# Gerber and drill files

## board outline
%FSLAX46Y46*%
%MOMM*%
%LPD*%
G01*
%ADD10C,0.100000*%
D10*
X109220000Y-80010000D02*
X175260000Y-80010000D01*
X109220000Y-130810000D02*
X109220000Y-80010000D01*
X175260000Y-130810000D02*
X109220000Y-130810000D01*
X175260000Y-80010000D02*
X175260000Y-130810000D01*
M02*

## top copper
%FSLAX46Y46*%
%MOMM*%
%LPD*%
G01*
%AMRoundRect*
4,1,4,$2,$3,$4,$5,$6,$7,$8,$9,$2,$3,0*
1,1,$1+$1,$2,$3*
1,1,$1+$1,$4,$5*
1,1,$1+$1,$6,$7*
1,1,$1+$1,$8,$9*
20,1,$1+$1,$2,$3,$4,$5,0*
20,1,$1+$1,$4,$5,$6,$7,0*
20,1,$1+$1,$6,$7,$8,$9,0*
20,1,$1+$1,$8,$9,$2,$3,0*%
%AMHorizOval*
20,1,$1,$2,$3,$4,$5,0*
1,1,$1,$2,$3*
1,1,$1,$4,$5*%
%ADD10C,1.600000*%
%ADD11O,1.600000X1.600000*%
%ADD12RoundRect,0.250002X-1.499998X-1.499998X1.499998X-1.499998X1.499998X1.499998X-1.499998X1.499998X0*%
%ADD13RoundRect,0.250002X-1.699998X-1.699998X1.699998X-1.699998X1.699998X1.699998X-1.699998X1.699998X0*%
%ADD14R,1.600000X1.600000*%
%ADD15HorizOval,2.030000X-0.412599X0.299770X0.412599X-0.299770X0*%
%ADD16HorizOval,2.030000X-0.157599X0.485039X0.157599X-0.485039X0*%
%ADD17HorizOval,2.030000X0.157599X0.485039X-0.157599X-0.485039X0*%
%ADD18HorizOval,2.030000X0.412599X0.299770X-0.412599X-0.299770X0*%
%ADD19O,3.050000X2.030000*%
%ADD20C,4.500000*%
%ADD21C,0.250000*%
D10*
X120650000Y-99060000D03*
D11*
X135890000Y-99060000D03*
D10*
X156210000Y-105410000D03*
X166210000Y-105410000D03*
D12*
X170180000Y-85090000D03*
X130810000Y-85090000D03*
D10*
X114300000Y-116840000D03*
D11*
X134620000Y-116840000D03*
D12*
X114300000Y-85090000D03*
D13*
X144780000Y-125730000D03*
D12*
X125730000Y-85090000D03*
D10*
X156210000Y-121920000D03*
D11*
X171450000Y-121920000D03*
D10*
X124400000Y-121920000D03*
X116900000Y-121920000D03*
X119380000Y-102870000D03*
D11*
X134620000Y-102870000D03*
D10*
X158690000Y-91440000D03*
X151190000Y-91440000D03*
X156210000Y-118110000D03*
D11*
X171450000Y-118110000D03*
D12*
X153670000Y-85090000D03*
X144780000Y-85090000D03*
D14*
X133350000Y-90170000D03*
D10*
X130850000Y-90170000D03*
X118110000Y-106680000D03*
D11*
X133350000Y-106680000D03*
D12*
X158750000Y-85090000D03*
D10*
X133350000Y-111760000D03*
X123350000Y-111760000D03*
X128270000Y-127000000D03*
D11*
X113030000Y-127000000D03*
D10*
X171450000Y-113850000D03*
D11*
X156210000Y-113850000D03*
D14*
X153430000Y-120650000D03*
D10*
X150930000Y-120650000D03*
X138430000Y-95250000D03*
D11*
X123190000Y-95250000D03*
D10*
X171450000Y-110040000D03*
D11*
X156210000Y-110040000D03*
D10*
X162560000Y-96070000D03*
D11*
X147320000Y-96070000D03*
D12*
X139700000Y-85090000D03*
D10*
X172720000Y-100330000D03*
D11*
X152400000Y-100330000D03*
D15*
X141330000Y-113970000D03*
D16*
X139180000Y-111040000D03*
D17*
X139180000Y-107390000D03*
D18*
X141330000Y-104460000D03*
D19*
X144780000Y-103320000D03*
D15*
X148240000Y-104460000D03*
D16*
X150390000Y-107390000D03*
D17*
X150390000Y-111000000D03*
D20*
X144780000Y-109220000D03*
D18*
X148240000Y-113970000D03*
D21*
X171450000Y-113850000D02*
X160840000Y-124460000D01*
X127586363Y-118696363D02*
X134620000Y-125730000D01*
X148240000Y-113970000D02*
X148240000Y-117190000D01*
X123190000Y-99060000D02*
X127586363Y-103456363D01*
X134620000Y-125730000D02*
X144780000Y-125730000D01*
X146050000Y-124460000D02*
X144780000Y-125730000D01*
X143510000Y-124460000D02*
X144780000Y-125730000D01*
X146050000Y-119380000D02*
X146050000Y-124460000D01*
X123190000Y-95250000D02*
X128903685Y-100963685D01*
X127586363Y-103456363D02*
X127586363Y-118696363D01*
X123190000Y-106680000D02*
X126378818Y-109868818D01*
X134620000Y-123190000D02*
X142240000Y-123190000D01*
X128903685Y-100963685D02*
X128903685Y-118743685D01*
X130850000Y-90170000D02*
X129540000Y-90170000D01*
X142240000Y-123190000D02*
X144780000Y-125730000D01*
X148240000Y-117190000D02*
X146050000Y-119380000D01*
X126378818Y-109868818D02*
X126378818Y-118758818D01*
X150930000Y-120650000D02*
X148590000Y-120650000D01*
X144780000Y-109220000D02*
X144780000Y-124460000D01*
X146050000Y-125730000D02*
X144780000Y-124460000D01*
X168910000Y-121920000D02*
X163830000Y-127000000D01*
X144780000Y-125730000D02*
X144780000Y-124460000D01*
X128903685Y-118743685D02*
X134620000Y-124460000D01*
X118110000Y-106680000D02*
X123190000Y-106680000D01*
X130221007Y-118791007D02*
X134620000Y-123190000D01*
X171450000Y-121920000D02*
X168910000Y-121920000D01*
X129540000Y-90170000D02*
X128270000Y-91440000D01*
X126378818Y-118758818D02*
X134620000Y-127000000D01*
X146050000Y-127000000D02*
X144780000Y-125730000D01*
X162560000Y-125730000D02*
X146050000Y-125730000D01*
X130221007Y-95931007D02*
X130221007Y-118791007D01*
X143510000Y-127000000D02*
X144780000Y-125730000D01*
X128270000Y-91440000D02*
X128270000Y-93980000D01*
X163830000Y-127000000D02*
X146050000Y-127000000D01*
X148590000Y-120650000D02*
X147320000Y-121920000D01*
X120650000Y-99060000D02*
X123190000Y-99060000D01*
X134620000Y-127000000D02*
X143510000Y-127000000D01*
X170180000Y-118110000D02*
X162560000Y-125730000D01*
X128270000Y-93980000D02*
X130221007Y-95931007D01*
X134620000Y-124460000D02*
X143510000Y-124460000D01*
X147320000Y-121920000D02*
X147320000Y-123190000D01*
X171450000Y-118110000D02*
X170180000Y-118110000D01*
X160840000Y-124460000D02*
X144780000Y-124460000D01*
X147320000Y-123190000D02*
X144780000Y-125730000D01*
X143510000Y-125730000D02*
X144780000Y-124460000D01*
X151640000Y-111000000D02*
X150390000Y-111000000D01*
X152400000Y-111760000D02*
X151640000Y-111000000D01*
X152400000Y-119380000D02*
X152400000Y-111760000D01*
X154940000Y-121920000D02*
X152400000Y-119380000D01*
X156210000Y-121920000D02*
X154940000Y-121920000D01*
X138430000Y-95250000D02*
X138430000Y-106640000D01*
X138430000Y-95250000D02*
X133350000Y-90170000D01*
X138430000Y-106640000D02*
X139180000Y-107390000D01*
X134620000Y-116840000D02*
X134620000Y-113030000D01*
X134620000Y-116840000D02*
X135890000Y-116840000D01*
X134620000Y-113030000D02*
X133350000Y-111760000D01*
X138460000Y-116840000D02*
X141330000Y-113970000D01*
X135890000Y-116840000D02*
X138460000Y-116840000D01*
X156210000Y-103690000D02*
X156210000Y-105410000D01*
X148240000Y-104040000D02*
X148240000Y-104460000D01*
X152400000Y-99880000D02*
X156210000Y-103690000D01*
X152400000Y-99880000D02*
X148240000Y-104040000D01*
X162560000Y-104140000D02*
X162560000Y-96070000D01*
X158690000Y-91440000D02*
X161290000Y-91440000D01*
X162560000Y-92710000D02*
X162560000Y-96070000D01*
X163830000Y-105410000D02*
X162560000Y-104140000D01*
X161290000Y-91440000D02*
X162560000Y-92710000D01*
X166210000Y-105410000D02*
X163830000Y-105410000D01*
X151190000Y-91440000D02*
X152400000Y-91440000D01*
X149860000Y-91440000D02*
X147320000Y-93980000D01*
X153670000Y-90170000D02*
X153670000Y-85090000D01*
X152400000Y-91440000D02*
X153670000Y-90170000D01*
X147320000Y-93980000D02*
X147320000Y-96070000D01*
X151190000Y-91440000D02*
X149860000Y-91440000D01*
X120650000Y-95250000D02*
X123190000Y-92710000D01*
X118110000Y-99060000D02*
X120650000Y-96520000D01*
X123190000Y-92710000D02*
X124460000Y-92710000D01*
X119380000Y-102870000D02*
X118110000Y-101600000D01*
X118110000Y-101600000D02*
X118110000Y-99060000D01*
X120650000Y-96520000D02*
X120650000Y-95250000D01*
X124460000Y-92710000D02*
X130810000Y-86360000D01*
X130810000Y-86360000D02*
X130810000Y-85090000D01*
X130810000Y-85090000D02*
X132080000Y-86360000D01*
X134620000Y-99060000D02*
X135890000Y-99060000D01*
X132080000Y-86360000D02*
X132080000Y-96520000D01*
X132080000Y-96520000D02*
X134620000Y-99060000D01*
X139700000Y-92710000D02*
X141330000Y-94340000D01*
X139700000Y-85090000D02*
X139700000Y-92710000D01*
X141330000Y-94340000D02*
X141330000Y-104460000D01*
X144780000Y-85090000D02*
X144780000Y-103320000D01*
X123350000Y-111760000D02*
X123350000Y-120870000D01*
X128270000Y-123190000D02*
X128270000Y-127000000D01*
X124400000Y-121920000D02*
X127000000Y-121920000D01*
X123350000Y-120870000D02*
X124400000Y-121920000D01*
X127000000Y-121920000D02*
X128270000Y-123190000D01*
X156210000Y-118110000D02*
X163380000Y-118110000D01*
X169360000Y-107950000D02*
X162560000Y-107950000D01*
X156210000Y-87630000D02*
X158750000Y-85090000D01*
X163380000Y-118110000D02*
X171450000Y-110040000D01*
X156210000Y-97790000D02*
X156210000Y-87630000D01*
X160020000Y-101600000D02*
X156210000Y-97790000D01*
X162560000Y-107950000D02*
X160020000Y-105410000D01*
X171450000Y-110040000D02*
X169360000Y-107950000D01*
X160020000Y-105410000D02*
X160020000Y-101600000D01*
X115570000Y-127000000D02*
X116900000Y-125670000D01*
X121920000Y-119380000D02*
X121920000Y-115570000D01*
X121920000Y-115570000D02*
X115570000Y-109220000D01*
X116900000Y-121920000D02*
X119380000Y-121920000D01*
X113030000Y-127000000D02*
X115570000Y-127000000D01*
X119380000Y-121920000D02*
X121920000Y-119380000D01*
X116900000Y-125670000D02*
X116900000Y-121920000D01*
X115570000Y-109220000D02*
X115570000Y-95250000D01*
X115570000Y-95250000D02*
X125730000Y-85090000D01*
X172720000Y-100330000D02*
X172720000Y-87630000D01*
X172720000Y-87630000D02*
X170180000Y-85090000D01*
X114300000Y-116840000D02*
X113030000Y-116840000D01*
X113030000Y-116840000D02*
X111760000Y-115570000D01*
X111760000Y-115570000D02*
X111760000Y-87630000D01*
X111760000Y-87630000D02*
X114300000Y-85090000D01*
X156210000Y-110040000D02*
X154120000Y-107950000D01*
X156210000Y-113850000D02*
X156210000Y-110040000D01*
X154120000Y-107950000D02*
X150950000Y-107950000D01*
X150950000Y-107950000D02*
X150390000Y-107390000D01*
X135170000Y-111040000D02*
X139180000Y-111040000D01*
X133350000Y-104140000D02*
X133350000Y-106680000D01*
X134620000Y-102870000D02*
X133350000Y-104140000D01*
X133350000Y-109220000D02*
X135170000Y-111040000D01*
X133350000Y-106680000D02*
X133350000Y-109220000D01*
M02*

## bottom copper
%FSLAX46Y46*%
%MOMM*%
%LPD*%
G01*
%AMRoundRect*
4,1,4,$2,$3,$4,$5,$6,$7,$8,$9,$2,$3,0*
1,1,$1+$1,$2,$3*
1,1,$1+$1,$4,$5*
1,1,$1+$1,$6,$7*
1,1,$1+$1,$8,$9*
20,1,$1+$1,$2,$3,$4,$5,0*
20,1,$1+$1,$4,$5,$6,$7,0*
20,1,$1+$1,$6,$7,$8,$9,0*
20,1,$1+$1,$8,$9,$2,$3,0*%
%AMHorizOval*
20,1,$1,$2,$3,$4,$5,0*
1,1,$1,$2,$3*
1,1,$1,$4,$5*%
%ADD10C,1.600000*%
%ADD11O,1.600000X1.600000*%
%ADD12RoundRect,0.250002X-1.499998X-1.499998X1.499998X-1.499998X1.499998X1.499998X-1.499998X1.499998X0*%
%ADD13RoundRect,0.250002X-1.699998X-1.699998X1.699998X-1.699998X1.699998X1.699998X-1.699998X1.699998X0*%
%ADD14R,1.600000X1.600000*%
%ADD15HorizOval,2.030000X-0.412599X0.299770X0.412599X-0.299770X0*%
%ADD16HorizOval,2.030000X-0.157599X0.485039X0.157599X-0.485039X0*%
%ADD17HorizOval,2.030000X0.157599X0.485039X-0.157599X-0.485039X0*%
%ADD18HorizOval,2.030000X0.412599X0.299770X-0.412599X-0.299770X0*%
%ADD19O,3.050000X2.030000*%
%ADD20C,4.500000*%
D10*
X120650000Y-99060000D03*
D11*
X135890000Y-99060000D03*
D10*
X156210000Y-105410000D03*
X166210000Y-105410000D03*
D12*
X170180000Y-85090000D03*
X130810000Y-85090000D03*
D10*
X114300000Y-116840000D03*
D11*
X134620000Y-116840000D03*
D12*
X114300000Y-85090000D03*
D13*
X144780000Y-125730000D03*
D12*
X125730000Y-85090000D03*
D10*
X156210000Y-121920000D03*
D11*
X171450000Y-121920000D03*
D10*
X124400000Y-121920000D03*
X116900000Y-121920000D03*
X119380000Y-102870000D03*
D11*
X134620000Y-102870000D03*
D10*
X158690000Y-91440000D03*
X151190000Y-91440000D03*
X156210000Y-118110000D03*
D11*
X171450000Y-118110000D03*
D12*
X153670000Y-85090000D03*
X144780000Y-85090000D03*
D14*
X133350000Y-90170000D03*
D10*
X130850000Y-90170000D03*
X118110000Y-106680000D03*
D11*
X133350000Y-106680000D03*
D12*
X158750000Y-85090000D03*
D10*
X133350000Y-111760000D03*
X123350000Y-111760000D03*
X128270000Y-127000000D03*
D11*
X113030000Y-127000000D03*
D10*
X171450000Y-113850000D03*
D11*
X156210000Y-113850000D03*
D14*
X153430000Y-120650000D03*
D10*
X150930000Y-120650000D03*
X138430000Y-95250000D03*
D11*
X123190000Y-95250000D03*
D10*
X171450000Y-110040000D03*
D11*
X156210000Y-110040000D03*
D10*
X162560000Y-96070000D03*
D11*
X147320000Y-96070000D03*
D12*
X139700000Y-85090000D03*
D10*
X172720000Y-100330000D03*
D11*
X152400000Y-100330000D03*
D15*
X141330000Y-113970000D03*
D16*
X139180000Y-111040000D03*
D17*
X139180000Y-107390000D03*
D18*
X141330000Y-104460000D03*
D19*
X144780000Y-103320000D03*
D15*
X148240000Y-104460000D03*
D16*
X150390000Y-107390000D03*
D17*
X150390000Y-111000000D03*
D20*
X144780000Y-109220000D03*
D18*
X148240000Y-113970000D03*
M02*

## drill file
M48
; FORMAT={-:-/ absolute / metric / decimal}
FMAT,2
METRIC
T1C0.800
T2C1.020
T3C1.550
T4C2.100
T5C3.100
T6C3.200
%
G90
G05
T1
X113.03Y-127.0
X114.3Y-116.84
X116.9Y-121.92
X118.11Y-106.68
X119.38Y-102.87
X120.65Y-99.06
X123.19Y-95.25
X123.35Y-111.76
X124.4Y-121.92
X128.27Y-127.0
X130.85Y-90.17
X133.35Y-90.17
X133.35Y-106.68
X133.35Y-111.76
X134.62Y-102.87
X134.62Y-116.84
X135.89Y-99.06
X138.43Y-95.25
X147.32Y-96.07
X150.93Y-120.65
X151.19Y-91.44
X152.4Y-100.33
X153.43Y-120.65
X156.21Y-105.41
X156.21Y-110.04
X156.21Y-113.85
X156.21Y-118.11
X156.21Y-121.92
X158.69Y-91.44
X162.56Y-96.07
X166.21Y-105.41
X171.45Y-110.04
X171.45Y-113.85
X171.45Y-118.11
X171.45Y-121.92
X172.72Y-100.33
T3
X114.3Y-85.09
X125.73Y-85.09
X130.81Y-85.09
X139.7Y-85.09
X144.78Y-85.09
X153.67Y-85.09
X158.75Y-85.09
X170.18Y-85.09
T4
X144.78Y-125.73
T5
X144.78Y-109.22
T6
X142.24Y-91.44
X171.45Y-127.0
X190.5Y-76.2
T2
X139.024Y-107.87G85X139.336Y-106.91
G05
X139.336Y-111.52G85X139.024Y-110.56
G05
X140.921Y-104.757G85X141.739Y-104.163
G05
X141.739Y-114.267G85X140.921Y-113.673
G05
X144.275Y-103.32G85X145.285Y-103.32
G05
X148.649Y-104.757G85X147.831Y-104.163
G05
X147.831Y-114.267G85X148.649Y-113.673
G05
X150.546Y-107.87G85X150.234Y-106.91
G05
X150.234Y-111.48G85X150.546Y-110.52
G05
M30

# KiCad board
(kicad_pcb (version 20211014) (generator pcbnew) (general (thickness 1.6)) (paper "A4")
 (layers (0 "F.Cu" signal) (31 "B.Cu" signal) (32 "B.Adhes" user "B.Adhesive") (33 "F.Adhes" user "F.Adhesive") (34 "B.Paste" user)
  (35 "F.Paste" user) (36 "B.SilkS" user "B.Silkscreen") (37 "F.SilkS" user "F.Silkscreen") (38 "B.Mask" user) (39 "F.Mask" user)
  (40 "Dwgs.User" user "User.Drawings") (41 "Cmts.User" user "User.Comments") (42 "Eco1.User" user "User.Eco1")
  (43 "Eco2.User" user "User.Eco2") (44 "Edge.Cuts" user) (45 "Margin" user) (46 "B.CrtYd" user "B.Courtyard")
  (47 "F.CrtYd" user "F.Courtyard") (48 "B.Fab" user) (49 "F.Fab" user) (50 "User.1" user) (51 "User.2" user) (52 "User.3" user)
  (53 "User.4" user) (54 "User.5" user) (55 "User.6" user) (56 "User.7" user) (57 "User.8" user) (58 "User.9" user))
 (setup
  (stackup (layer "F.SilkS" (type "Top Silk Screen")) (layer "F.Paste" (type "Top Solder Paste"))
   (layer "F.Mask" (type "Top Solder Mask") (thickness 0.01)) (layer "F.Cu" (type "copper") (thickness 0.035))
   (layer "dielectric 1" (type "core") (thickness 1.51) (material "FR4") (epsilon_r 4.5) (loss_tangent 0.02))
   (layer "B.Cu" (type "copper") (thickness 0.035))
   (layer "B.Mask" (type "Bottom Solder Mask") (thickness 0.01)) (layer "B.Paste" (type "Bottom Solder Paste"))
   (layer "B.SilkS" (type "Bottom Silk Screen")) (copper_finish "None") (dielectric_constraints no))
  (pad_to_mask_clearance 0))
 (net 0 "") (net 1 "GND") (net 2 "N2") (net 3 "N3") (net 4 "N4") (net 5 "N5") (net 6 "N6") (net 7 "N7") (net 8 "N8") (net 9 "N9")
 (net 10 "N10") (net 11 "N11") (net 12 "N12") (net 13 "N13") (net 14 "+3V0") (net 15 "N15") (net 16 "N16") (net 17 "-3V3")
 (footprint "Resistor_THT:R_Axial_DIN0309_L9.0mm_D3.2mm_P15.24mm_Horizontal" (layer "F.Cu") (at 120.65 99.06)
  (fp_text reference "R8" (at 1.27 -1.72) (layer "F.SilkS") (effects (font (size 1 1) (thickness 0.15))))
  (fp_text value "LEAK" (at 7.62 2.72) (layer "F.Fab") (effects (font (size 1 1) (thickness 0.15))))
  (pad "1" thru_hole circle (at 0 0) (size 1.6 1.6) (drill 0.8) (layers *.Cu *.Mask) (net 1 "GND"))
  (pad "2" thru_hole oval (at 15.24 0) (size 1.6 1.6) (drill 0.8) (layers *.Cu *.Mask) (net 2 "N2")))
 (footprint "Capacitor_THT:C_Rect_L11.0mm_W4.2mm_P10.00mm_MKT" (layer "F.Cu") (at 156.21 105.41)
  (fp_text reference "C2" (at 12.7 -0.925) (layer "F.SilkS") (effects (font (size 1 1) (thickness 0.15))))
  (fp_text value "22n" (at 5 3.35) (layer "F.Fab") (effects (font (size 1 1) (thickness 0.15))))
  (pad "1" thru_hole circle (at 0 0) (size 1.6 1.6) (drill 0.8) (layers *.Cu *.Mask) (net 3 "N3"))
  (pad "2" thru_hole circle (at 10 0) (size 1.6 1.6) (drill 0.8) (layers *.Cu *.Mask) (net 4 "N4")))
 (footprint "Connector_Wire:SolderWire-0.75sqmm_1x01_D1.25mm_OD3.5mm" (layer "F.Cu") (at 170.18 85.09)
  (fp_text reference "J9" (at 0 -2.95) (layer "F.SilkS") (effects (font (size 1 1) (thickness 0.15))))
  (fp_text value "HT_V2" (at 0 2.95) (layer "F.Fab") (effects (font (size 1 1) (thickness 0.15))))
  (pad "1" thru_hole roundrect (at 0 0) (size 3.5 3.5) (drill 1.55) (layers *.Cu *.Mask) (roundrect_rratio 0.071429) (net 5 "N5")))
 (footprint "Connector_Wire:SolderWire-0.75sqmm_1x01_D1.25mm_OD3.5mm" (layer "F.Cu") (at 130.81 85.09)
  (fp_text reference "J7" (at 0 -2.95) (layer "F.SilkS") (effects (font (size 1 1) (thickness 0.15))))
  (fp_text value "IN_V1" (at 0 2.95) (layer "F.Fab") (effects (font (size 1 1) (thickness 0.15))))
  (pad "1" thru_hole roundrect (at 0 0) (size 3.5 3.5) (drill 1.55) (layers *.Cu *.Mask) (roundrect_rratio 0.071429) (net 2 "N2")))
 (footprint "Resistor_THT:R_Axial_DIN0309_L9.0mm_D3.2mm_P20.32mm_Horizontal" (layer "F.Cu") (at 114.3 116.84)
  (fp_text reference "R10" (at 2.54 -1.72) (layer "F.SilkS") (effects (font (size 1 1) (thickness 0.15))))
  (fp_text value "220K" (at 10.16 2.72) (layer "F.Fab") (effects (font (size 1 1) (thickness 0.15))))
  (pad "1" thru_hole circle (at 0 0) (size 1.6 1.6) (drill 0.8) (layers *.Cu *.Mask) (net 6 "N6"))
  (pad "2" thru_hole oval (at 20.32 0) (size 1.6 1.6) (drill 0.8) (layers *.Cu *.Mask) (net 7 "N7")))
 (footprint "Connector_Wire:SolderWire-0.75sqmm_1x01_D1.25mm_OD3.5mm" (layer "F.Cu") (at 114.3 85.09)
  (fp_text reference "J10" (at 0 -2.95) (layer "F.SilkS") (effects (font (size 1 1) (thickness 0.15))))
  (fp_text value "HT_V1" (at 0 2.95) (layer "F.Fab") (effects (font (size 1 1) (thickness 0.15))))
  (pad "1" thru_hole roundrect (at 0 0) (size 3.5 3.5) (drill 1.55) (layers *.Cu *.Mask) (roundrect_rratio 0.071429) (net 6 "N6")))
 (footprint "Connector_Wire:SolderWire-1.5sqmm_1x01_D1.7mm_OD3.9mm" (layer "F.Cu") (at 144.78 125.73)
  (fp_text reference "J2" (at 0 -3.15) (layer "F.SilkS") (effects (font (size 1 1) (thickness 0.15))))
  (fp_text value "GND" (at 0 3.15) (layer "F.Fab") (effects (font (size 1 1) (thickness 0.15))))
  (pad "1" thru_hole roundrect (at 0 0) (size 3.9 3.9) (drill 2.1) (layers *.Cu *.Mask) (roundrect_rratio 0.064103) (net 1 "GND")))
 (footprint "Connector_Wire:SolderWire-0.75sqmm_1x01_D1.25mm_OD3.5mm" (layer "F.Cu") (at 125.73 85.09)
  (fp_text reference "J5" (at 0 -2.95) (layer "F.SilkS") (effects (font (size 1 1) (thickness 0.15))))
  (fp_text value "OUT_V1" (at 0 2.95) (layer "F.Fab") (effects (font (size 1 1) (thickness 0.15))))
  (pad "1" thru_hole roundrect (at 0 0) (size 3.5 3.5) (drill 1.55) (layers *.Cu *.Mask) (roundrect_rratio 0.071429) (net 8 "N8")))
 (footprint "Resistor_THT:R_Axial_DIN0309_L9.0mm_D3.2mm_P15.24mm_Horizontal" (layer "F.Cu") (at 156.21 121.92)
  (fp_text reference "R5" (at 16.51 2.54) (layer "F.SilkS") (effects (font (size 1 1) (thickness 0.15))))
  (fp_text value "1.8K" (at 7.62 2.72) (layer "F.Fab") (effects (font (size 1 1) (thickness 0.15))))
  (pad "1" thru_hole circle (at 0 0) (size 1.6 1.6) (drill 0.8) (layers *.Cu *.Mask) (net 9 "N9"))
  (pad "2" thru_hole oval (at 15.24 0) (size 1.6 1.6) (drill 0.8) (layers *.Cu *.Mask) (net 1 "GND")))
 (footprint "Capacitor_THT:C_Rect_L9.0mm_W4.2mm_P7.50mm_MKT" (layer "F.Cu") (at 124.4 121.92 180)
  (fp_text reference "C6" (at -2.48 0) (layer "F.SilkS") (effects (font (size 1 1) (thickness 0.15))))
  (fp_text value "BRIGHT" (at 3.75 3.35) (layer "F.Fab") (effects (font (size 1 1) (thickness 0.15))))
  (pad "1" thru_hole circle (at 0 0 180) (size 1.6 1.6) (drill 0.8) (layers *.Cu *.Mask) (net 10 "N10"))
  (pad "2" thru_hole circle (at 7.5 0 180) (size 1.6 1.6) (drill 0.8) (layers *.Cu *.Mask) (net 8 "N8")))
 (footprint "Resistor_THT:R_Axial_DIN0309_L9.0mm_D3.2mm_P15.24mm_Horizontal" (layer "F.Cu") (at 119.38 102.87)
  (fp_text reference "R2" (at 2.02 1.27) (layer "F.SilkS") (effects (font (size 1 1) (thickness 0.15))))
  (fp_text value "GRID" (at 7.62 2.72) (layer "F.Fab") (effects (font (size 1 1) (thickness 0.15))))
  (pad "1" thru_hole circle (at 0 0) (size 1.6 1.6) (drill 0.8) (layers *.Cu *.Mask) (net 2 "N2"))
  (pad "2" thru_hole oval (at 15.24 0) (size 1.6 1.6) (drill 0.8) (layers *.Cu *.Mask) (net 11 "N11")))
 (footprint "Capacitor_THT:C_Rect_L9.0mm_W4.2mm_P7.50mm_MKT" (layer "F.Cu") (at 158.69 91.44 180)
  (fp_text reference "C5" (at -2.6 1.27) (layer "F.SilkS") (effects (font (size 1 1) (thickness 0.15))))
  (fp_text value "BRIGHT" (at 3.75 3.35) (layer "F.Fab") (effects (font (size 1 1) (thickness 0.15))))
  (pad "1" thru_hole circle (at 0 0 180) (size 1.6 1.6) (drill 0.8) (layers *.Cu *.Mask) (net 4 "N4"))
  (pad "2" thru_hole circle (at 7.5 0 180) (size 1.6 1.6) (drill 0.8) (layers *.Cu *.Mask) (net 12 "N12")))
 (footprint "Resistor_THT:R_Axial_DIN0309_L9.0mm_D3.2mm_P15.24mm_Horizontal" (layer "F.Cu") (at 156.21 118.11)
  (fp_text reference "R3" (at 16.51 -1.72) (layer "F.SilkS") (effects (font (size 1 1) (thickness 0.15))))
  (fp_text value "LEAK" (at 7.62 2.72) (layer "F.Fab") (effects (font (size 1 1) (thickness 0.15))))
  (pad "1" thru_hole circle (at 0 0) (size 1.6 1.6) (drill 0.8) (layers *.Cu *.Mask) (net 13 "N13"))
  (pad "2" thru_hole oval (at 15.24 0) (size 1.6 1.6) (drill 0.8) (layers *.Cu *.Mask) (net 1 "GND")))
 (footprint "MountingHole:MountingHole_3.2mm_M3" (layer "F.Cu") (at 171.45 127)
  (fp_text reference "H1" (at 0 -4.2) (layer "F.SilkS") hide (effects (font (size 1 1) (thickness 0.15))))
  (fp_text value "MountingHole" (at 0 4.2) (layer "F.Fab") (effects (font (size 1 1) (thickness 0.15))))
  (pad "" np_thru_hole circle (at 0 0) (size 3.2 3.2) (drill 3.2) (layers *.Cu *.Mask)))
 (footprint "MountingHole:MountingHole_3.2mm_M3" (layer "F.Cu") (at 190.5 76.2)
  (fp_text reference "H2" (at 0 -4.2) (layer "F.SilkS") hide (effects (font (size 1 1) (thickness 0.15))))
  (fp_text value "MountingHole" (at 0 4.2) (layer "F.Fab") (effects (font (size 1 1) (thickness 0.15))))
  (pad "" np_thru_hole circle (at 0 0) (size 3.2 3.2) (drill 3.2) (layers *.Cu *.Mask)))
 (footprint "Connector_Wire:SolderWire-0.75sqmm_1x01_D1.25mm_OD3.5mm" (layer "F.Cu") (at 153.67 85.09)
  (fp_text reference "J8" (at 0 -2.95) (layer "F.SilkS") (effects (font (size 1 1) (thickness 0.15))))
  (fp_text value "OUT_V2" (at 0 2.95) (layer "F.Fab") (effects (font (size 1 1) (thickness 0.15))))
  (pad "1" thru_hole roundrect (at 0 0) (size 3.5 3.5) (drill 1.55) (layers *.Cu *.Mask) (roundrect_rratio 0.071429) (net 12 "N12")))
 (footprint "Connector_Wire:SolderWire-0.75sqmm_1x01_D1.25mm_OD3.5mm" (layer "F.Cu") (at 144.78 85.09)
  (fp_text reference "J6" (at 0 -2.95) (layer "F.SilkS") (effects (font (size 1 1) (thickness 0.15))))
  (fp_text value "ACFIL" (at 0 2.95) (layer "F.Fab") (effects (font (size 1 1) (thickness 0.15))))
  (pad "1" thru_hole roundrect (at 0 0) (size 3.5 3.5) (drill 1.55) (layers *.Cu *.Mask) (roundrect_rratio 0.071429) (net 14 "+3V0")))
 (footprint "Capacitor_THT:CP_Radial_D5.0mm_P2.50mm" (layer "F.Cu") (at 133.35 90.17 180)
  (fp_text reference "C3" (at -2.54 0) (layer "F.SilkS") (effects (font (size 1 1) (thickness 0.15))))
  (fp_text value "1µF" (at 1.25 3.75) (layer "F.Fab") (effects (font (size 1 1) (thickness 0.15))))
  (pad "1" thru_hole rect (at 0 0 180) (size 1.6 1.6) (drill 0.8) (layers *.Cu *.Mask) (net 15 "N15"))
  (pad "2" thru_hole circle (at 2.5 0 180) (size 1.6 1.6) (drill 0.8) (layers *.Cu *.Mask) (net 1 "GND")))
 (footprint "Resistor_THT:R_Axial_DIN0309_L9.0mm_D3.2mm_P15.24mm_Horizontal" (layer "F.Cu") (at 118.11 106.68)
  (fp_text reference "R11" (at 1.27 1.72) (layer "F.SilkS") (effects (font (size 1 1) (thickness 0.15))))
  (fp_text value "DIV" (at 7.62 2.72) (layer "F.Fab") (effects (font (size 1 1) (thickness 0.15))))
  (pad "1" thru_hole circle (at 0 0) (size 1.6 1.6) (drill 0.8) (layers *.Cu *.Mask) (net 1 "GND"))
  (pad "2" thru_hole oval (at 15.24 0) (size 1.6 1.6) (drill 0.8) (layers *.Cu *.Mask) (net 11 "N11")))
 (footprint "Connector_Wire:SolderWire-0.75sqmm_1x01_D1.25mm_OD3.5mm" (layer "F.Cu") (at 158.75 85.09)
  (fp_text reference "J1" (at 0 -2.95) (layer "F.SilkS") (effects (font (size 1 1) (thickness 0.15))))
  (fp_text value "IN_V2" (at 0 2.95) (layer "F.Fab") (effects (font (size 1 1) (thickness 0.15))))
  (pad "1" thru_hole roundrect (at 0 0) (size 3.5 3.5) (drill 1.55) (layers *.Cu *.Mask) (roundrect_rratio 0.071429) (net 13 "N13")))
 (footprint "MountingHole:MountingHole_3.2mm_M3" (layer "F.Cu") (at 142.24 91.44)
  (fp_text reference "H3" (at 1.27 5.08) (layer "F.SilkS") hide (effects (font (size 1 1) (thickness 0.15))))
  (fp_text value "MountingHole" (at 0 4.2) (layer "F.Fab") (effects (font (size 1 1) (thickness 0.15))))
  (pad "" np_thru_hole circle (at 0 0) (size 3.2 3.2) (drill 3.2) (layers *.Cu *.Mask)))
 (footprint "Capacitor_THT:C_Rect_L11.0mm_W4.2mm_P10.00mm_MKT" (layer "F.Cu") (at 133.35 111.76 180)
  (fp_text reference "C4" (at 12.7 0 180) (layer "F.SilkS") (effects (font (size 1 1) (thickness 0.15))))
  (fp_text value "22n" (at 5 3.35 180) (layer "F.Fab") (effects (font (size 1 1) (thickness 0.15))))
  (pad "1" thru_hole circle (at 0 0 180) (size 1.6 1.6) (drill 0.8) (layers *.Cu *.Mask) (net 7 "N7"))
  (pad "2" thru_hole circle (at 10 0 180) (size 1.6 1.6) (drill 0.8) (layers *.Cu *.Mask) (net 10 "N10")))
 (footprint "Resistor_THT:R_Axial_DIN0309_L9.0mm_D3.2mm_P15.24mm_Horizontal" (layer "F.Cu") (at 128.27 127 180)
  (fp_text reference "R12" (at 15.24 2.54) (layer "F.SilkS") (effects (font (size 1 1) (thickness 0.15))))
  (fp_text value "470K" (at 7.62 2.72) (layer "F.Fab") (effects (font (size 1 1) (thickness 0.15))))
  (pad "1" thru_hole circle (at 0 0 180) (size 1.6 1.6) (drill 0.8) (layers *.Cu *.Mask) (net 10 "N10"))
  (pad "2" thru_hole oval (at 15.24 0 180) (size 1.6 1.6) (drill 0.8) (layers *.Cu *.Mask) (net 8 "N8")))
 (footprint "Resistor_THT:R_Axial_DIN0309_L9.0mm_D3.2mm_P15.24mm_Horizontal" (layer "F.Cu") (at 171.45 113.85 180)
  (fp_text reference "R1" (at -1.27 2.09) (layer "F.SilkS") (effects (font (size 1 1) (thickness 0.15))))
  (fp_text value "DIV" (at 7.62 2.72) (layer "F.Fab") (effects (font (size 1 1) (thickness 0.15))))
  (pad "1" thru_hole circle (at 0 0 180) (size 1.6 1.6) (drill 0.8) (layers *.Cu *.Mask) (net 1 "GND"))
  (pad "2" thru_hole oval (at 15.24 0 180) (size 1.6 1.6) (drill 0.8) (layers *.Cu *.Mask) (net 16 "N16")))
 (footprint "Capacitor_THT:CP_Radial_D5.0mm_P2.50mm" (layer "F.Cu") (at 153.43 120.65 180)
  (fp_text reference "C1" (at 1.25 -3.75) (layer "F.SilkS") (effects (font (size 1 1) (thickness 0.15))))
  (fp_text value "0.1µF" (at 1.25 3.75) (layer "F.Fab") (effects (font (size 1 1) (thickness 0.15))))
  (pad "1" thru_hole rect (at 0 0 180) (size 1.6 1.6) (drill 0.8) (layers *.Cu *.Mask) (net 9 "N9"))
  (pad "2" thru_hole circle (at 2.5 0 180) (size 1.6 1.6) (drill 0.8) (layers *.Cu *.Mask) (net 1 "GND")))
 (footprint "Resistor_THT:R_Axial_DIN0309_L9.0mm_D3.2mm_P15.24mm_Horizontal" (layer "F.Cu") (at 138.43 95.25 180)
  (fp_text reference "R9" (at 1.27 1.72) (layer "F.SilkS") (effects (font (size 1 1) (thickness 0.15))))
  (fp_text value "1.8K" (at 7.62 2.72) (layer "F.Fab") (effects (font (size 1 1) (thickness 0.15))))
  (pad "1" thru_hole circle (at 0 0 180) (size 1.6 1.6) (drill 0.8) (layers *.Cu *.Mask) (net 15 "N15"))
  (pad "2" thru_hole oval (at 15.24 0 180) (size 1.6 1.6) (drill 0.8) (layers *.Cu *.Mask) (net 1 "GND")))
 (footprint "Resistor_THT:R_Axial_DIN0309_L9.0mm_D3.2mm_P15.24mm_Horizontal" (layer "F.Cu") (at 171.45 110.04 180)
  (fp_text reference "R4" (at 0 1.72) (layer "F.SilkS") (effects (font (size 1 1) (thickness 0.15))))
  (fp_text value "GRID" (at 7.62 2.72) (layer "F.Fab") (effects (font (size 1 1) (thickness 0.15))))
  (pad "1" thru_hole circle (at 0 0 180) (size 1.6 1.6) (drill 0.8) (layers *.Cu *.Mask) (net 13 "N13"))
  (pad "2" thru_hole oval (at 15.24 0 180) (size 1.6 1.6) (drill 0.8) (layers *.Cu *.Mask) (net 16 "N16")))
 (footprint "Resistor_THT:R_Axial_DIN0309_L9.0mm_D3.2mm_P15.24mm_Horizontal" (layer "F.Cu") (at 162.56 96.07 180)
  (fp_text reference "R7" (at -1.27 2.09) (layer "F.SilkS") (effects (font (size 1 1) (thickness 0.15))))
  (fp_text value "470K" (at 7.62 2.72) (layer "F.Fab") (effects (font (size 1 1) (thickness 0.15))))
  (pad "1" thru_hole circle (at 0 0 180) (size 1.6 1.6) (drill 0.8) (layers *.Cu *.Mask) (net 4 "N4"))
  (pad "2" thru_hole oval (at 15.24 0 180) (size 1.6 1.6) (drill 0.8) (layers *.Cu *.Mask) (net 12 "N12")))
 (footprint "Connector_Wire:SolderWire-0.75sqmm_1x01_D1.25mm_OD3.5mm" (layer "F.Cu") (at 139.7 85.09)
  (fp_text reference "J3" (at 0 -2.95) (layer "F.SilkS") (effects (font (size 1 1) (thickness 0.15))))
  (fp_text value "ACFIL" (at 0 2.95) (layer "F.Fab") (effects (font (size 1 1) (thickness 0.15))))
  (pad "1" thru_hole roundrect (at 0 0) (size 3.5 3.5) (drill 1.55) (layers *.Cu *.Mask) (roundrect_rratio 0.071429) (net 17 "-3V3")))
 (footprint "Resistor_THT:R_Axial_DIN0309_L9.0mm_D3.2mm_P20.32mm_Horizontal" (layer "F.Cu") (at 172.72 100.33 180)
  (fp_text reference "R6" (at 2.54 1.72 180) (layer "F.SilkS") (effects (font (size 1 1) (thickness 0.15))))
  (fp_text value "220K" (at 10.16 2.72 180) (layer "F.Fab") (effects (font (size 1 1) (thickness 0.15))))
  (pad "1" thru_hole circle (at 0 0 180) (size 1.6 1.6) (drill 0.8) (layers *.Cu *.Mask) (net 5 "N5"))
  (pad "2" thru_hole oval (at 20.32 0 180) (size 1.6 1.6) (drill 0.8) (layers *.Cu *.Mask) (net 3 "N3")))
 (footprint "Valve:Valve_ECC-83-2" (layer "B.Cu") (at 141.33 113.97 180)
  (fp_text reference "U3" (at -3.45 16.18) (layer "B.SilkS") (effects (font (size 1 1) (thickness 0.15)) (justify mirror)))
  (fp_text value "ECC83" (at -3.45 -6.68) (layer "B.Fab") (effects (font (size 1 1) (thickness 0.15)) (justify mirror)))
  (pad "1" thru_hole oval (at 0 0 234) (size 2.03 3.05) (drill oval 1.02 2.03) (layers *.Cu *.Mask) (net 7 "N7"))
  (pad "2" thru_hole oval (at 2.15 2.93 198) (size 2.03 3.05) (drill oval 1.02 2.03) (layers *.Cu *.Mask) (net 11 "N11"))
  (pad "3" thru_hole oval (at 2.15 6.58 162) (size 2.03 3.05) (drill oval 1.02 2.03) (layers *.Cu *.Mask) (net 15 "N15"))
  (pad "4" thru_hole oval (at 0 9.51 126) (size 2.03 3.05) (drill oval 1.02 2.03) (layers *.Cu *.Mask) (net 17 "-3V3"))
  (pad "5" thru_hole oval (at -3.45 10.65 90) (size 2.03 3.05) (drill oval 1.02 2.03) (layers *.Cu *.Mask) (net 14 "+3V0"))
  (pad "6" thru_hole oval (at -6.91 9.51 234) (size 2.03 3.05) (drill oval 1.02 2.03) (layers *.Cu *.Mask) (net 3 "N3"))
  (pad "7" thru_hole oval (at -9.06 6.58 198) (size 2.03 3.05) (drill oval 1.02 2.03) (layers *.Cu *.Mask) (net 16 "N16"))
  (pad "8" thru_hole oval (at -9.06 2.97 162) (size 2.03 3.05) (drill oval 1.02 2.03) (layers *.Cu *.Mask) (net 9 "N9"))
  (pad "9" thru_hole circle (at -3.45 4.75 180) (size 4.5 4.5) (drill 3.1) (layers *.Cu *.Mask) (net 1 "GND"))
  (pad "9" thru_hole oval (at -6.91 0 126) (size 2.03 3.05) (drill oval 1.02 2.03) (layers *.Cu *.Mask) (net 1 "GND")))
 (gr_line (start 109.22 80.01) (end 175.26 80.01) (layer "Edge.Cuts") (width 0.1))
 (gr_line (start 109.22 130.81) (end 109.22 80.01) (layer "Edge.Cuts") (width 0.1))
 (gr_line (start 175.26 130.81) (end 109.22 130.81) (layer "Edge.Cuts") (width 0.1))
 (gr_line (start 175.26 80.01) (end 175.26 130.81) (layer "Edge.Cuts") (width 0.1))
 (segment (start 171.45 113.85) (end 160.84 124.46) (width 0.25) (layer "F.Cu") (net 1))
 (segment (start 127.586363 118.696363) (end 134.62 125.73) (width 0.25) (layer "F.Cu") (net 1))
 (segment (start 148.24 113.97) (end 148.24 117.19) (width 0.25) (layer "F.Cu") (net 1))
 (segment (start 123.19 99.06) (end 127.586363 103.456363) (width 0.25) (layer "F.Cu") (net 1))
 (segment (start 134.62 125.73) (end 144.78 125.73) (width 0.25) (layer "F.Cu") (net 1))
 (segment (start 146.05 124.46) (end 144.78 125.73) (width 0.25) (layer "F.Cu") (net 1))
 (segment (start 143.51 124.46) (end 144.78 125.73) (width 0.25) (layer "F.Cu") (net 1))
 (segment (start 146.05 119.38) (end 146.05 124.46) (width 0.25) (layer "F.Cu") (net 1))
 (segment (start 123.19 95.25) (end 128.903685 100.963685) (width 0.25) (layer "F.Cu") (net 1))
 (segment (start 127.586363 103.456363) (end 127.586363 118.696363) (width 0.25) (layer "F.Cu") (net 1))
 (segment (start 123.19 106.68) (end 126.378818 109.868818) (width 0.25) (layer "F.Cu") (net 1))
 (segment (start 134.62 123.19) (end 142.24 123.19) (width 0.25) (layer "F.Cu") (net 1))
 (segment (start 128.903685 100.963685) (end 128.903685 118.743685) (width 0.25) (layer "F.Cu") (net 1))
 (segment (start 130.85 90.17) (end 129.54 90.17) (width 0.25) (layer "F.Cu") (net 1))
 (segment (start 142.24 123.19) (end 144.78 125.73) (width 0.25) (layer "F.Cu") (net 1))
 (segment (start 148.24 117.19) (end 146.05 119.38) (width 0.25) (layer "F.Cu") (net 1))
 (segment (start 126.378818 109.868818) (end 126.378818 118.758818) (width 0.25) (layer "F.Cu") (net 1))
 (segment (start 150.93 120.65) (end 148.59 120.65) (width 0.25) (layer "F.Cu") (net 1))
 (segment (start 144.78 109.22) (end 144.78 124.46) (width 0.25) (layer "F.Cu") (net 1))
 (segment (start 146.05 125.73) (end 144.78 124.46) (width 0.25) (layer "F.Cu") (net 1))
 (segment (start 168.91 121.92) (end 163.83 127) (width 0.25) (layer "F.Cu") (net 1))
 (segment (start 144.78 125.73) (end 144.78 124.46) (width 0.25) (layer "F.Cu") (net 1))
 (segment (start 128.903685 118.743685) (end 134.62 124.46) (width 0.25) (layer "F.Cu") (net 1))
 (segment (start 118.11 106.68) (end 123.19 106.68) (width 0.25) (layer "F.Cu") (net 1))
 (segment (start 130.221007 118.791007) (end 134.62 123.19) (width 0.25) (layer "F.Cu") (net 1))
 (segment (start 171.45 121.92) (end 168.91 121.92) (width 0.25) (layer "F.Cu") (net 1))
 (segment (start 129.54 90.17) (end 128.27 91.44) (width 0.25) (layer "F.Cu") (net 1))
 (segment (start 126.378818 118.758818) (end 134.62 127) (width 0.25) (layer "F.Cu") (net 1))
 (segment (start 146.05 127) (end 144.78 125.73) (width 0.25) (layer "F.Cu") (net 1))
 (segment (start 162.56 125.73) (end 146.05 125.73) (width 0.25) (layer "F.Cu") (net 1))
 (segment (start 130.221007 95.931007) (end 130.221007 118.791007) (width 0.25) (layer "F.Cu") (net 1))
 (segment (start 143.51 127) (end 144.78 125.73) (width 0.25) (layer "F.Cu") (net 1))
 (segment (start 128.27 91.44) (end 128.27 93.98) (width 0.25) (layer "F.Cu") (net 1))
 (segment (start 163.83 127) (end 146.05 127) (width 0.25) (layer "F.Cu") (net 1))
 (segment (start 148.59 120.65) (end 147.32 121.92) (width 0.25) (layer "F.Cu") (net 1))
 (segment (start 120.65 99.06) (end 123.19 99.06) (width 0.25) (layer "F.Cu") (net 1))
 (segment (start 134.62 127) (end 143.51 127) (width 0.25) (layer "F.Cu") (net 1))
 (segment (start 170.18 118.11) (end 162.56 125.73) (width 0.25) (layer "F.Cu") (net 1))
 (segment (start 128.27 93.98) (end 130.221007 95.931007) (width 0.25) (layer "F.Cu") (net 1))
 (segment (start 134.62 124.46) (end 143.51 124.46) (width 0.25) (layer "F.Cu") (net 1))
 (segment (start 147.32 121.92) (end 147.32 123.19) (width 0.25) (layer "F.Cu") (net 1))
 (segment (start 171.45 118.11) (end 170.18 118.11) (width 0.25) (layer "F.Cu") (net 1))
 (segment (start 160.84 124.46) (end 144.78 124.46) (width 0.25) (layer "F.Cu") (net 1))
 (segment (start 147.32 123.19) (end 144.78 125.73) (width 0.25) (layer "F.Cu") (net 1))
 (segment (start 143.51 125.73) (end 144.78 124.46) (width 0.25) (layer "F.Cu") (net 1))
 (segment (start 151.64 111) (end 150.39 111) (width 0.25) (layer "F.Cu") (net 9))
 (segment (start 152.4 111.76) (end 151.64 111) (width 0.25) (layer "F.Cu") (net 9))
 (segment (start 152.4 119.38) (end 152.4 111.76) (width 0.25) (layer "F.Cu") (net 9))
 (segment (start 154.94 121.92) (end 152.4 119.38) (width 0.25) (layer "F.Cu") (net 9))
 (segment (start 156.21 121.92) (end 154.94 121.92) (width 0.25) (layer "F.Cu") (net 9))
 (segment (start 138.43 95.25) (end 138.43 106.64) (width 0.25) (layer "F.Cu") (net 15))
 (segment (start 138.43 95.25) (end 133.35 90.17) (width 0.25) (layer "F.Cu") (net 15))
 (segment (start 138.43 106.64) (end 139.18 107.39) (width 0.25) (layer "F.Cu") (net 15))
 (segment (start 134.62 116.84) (end 134.62 113.03) (width 0.25) (layer "F.Cu") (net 7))
 (segment (start 134.62 116.84) (end 135.89 116.84) (width 0.25) (layer "F.Cu") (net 7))
 (segment (start 134.62 113.03) (end 133.35 111.76) (width 0.25) (layer "F.Cu") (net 7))
 (segment (start 138.46 116.84) (end 141.33 113.97) (width 0.25) (layer "F.Cu") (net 7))
 (segment (start 135.89 116.84) (end 138.46 116.84) (width 0.25) (layer "F.Cu") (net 7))
 (segment (start 156.21 103.69) (end 156.21 105.41) (width 0.25) (layer "F.Cu") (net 3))
 (segment (start 148.24 104.04) (end 148.24 104.46) (width 0.25) (layer "F.Cu") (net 3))
 (segment (start 152.4 99.88) (end 156.21 103.69) (width 0.25) (layer "F.Cu") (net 3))
 (segment (start 152.4 99.88) (end 148.24 104.04) (width 0.25) (layer "F.Cu") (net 3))
 (segment (start 162.56 104.14) (end 162.56 96.07) (width 0.25) (layer "F.Cu") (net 4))
 (segment (start 158.69 91.44) (end 161.29 91.44) (width 0.25) (layer "F.Cu") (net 4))
 (segment (start 162.56 92.71) (end 162.56 96.07) (width 0.25) (layer "F.Cu") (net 4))
 (segment (start 163.83 105.41) (end 162.56 104.14) (width 0.25) (layer "F.Cu") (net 4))
 (segment (start 161.29 91.44) (end 162.56 92.71) (width 0.25) (layer "F.Cu") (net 4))
 (segment (start 166.21 105.41) (end 163.83 105.41) (width 0.25) (layer "F.Cu") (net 4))
 (segment (start 151.19 91.44) (end 152.4 91.44) (width 0.25) (layer "F.Cu") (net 12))
 (segment (start 149.86 91.44) (end 147.32 93.98) (width 0.25) (layer "F.Cu") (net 12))
 (segment (start 153.67 90.17) (end 153.67 85.09) (width 0.25) (layer "F.Cu") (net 12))
 (segment (start 152.4 91.44) (end 153.67 90.17) (width 0.25) (layer "F.Cu") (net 12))
 (segment (start 147.32 93.98) (end 147.32 96.07) (width 0.25) (layer "F.Cu") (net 12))
 (segment (start 151.19 91.44) (end 149.86 91.44) (width 0.25) (layer "F.Cu") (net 12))
 (segment (start 120.65 95.25) (end 123.19 92.71) (width 0.25) (layer "F.Cu") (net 2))
 (segment (start 118.11 99.06) (end 120.65 96.52) (width 0.25) (layer "F.Cu") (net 2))
 (segment (start 123.19 92.71) (end 124.46 92.71) (width 0.25) (layer "F.Cu") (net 2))
 (segment (start 119.38 102.87) (end 118.11 101.6) (width 0.25) (layer "F.Cu") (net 2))
 (segment (start 118.11 101.6) (end 118.11 99.06) (width 0.25) (layer "F.Cu") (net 2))
 (segment (start 120.65 96.52) (end 120.65 95.25) (width 0.25) (layer "F.Cu") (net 2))
 (segment (start 124.46 92.71) (end 130.81 86.36) (width 0.25) (layer "F.Cu") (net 2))
 (segment (start 130.81 86.36) (end 130.81 85.09) (width 0.25) (layer "F.Cu") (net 2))
 (segment (start 130.81 85.09) (end 132.08 86.36) (width 0.25) (layer "F.Cu") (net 2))
 (segment (start 134.62 99.06) (end 135.89 99.06) (width 0.25) (layer "F.Cu") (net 2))
 (segment (start 132.08 86.36) (end 132.08 96.52) (width 0.25) (layer "F.Cu") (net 2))
 (segment (start 132.08 96.52) (end 134.62 99.06) (width 0.25) (layer "F.Cu") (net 2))
 (segment (start 139.7 92.71) (end 141.33 94.34) (width 0.25) (layer "F.Cu") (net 17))
 (segment (start 139.7 85.09) (end 139.7 92.71) (width 0.25) (layer "F.Cu") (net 17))
 (segment (start 141.33 94.34) (end 141.33 104.46) (width 0.25) (layer "F.Cu") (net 17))
 (segment (start 144.78 85.09) (end 144.78 103.32) (width 0.25) (layer "F.Cu") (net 14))
 (segment (start 123.35 111.76) (end 123.35 120.87) (width 0.25) (layer "F.Cu") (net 10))
 (segment (start 128.27 123.19) (end 128.27 127) (width 0.25) (layer "F.Cu") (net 10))
 (segment (start 124.4 121.92) (end 127 121.92) (width 0.25) (layer "F.Cu") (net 10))
 (segment (start 123.35 120.87) (end 124.4 121.92) (width 0.25) (layer "F.Cu") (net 10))
 (segment (start 127 121.92) (end 128.27 123.19) (width 0.25) (layer "F.Cu") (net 10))
 (segment (start 156.21 118.11) (end 163.38 118.11) (width 0.25) (layer "F.Cu") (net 13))
 (segment (start 169.36 107.95) (end 162.56 107.95) (width 0.25) (layer "F.Cu") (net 13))
 (segment (start 156.21 87.63) (end 158.75 85.09) (width 0.25) (layer "F.Cu") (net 13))
 (segment (start 163.38 118.11) (end 171.45 110.04) (width 0.25) (layer "F.Cu") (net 13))
 (segment (start 156.21 97.79) (end 156.21 87.63) (width 0.25) (layer "F.Cu") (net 13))
 (segment (start 160.02 101.6) (end 156.21 97.79) (width 0.25) (layer "F.Cu") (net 13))
 (segment (start 162.56 107.95) (end 160.02 105.41) (width 0.25) (layer "F.Cu") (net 13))
 (segment (start 171.45 110.04) (end 169.36 107.95) (width 0.25) (layer "F.Cu") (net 13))
 (segment (start 160.02 105.41) (end 160.02 101.6) (width 0.25) (layer "F.Cu") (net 13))
 (segment (start 115.57 127) (end 116.9 125.67) (width 0.25) (layer "F.Cu") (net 8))
 (segment (start 121.92 119.38) (end 121.92 115.57) (width 0.25) (layer "F.Cu") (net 8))
 (segment (start 121.92 115.57) (end 115.57 109.22) (width 0.25) (layer "F.Cu") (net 8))
 (segment (start 116.9 121.92) (end 119.38 121.92) (width 0.25) (layer "F.Cu") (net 8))
 (segment (start 113.03 127) (end 115.57 127) (width 0.25) (layer "F.Cu") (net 8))
 (segment (start 119.38 121.92) (end 121.92 119.38) (width 0.25) (layer "F.Cu") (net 8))
 (segment (start 116.9 125.67) (end 116.9 121.92) (width 0.25) (layer "F.Cu") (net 8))
 (segment (start 115.57 109.22) (end 115.57 95.25) (width 0.25) (layer "F.Cu") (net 8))
 (segment (start 115.57 95.25) (end 125.73 85.09) (width 0.25) (layer "F.Cu") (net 8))
 (segment (start 172.72 100.33) (end 172.72 87.63) (width 0.25) (layer "F.Cu") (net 5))
 (segment (start 172.72 87.63) (end 170.18 85.09) (width 0.25) (layer "F.Cu") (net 5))
 (segment (start 114.3 116.84) (end 113.03 116.84) (width 0.25) (layer "F.Cu") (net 6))
 (segment (start 113.03 116.84) (end 111.76 115.57) (width 0.25) (layer "F.Cu") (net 6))
 (segment (start 111.76 115.57) (end 111.76 87.63) (width 0.25) (layer "F.Cu") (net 6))
 (segment (start 111.76 87.63) (end 114.3 85.09) (width 0.25) (layer "F.Cu") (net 6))
 (segment (start 156.21 110.04) (end 154.12 107.95) (width 0.25) (layer "F.Cu") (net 16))
 (segment (start 156.21 113.85) (end 156.21 110.04) (width 0.25) (layer "F.Cu") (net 16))
 (segment (start 154.12 107.95) (end 150.95 107.95) (width 0.25) (layer "F.Cu") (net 16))
 (segment (start 150.95 107.95) (end 150.39 107.39) (width 0.25) (layer "F.Cu") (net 16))
 (segment (start 135.17 111.04) (end 139.18 111.04) (width 0.25) (layer "F.Cu") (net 11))
 (segment (start 133.35 104.14) (end 133.35 106.68) (width 0.25) (layer "F.Cu") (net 11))
 (segment (start 134.62 102.87) (end 133.35 104.14) (width 0.25) (layer "F.Cu") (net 11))
 (segment (start 133.35 109.22) (end 135.17 111.04) (width 0.25) (layer "F.Cu") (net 11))
 (segment (start 133.35 106.68) (end 133.35 109.22) (width 0.25) (layer "F.Cu") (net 11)))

